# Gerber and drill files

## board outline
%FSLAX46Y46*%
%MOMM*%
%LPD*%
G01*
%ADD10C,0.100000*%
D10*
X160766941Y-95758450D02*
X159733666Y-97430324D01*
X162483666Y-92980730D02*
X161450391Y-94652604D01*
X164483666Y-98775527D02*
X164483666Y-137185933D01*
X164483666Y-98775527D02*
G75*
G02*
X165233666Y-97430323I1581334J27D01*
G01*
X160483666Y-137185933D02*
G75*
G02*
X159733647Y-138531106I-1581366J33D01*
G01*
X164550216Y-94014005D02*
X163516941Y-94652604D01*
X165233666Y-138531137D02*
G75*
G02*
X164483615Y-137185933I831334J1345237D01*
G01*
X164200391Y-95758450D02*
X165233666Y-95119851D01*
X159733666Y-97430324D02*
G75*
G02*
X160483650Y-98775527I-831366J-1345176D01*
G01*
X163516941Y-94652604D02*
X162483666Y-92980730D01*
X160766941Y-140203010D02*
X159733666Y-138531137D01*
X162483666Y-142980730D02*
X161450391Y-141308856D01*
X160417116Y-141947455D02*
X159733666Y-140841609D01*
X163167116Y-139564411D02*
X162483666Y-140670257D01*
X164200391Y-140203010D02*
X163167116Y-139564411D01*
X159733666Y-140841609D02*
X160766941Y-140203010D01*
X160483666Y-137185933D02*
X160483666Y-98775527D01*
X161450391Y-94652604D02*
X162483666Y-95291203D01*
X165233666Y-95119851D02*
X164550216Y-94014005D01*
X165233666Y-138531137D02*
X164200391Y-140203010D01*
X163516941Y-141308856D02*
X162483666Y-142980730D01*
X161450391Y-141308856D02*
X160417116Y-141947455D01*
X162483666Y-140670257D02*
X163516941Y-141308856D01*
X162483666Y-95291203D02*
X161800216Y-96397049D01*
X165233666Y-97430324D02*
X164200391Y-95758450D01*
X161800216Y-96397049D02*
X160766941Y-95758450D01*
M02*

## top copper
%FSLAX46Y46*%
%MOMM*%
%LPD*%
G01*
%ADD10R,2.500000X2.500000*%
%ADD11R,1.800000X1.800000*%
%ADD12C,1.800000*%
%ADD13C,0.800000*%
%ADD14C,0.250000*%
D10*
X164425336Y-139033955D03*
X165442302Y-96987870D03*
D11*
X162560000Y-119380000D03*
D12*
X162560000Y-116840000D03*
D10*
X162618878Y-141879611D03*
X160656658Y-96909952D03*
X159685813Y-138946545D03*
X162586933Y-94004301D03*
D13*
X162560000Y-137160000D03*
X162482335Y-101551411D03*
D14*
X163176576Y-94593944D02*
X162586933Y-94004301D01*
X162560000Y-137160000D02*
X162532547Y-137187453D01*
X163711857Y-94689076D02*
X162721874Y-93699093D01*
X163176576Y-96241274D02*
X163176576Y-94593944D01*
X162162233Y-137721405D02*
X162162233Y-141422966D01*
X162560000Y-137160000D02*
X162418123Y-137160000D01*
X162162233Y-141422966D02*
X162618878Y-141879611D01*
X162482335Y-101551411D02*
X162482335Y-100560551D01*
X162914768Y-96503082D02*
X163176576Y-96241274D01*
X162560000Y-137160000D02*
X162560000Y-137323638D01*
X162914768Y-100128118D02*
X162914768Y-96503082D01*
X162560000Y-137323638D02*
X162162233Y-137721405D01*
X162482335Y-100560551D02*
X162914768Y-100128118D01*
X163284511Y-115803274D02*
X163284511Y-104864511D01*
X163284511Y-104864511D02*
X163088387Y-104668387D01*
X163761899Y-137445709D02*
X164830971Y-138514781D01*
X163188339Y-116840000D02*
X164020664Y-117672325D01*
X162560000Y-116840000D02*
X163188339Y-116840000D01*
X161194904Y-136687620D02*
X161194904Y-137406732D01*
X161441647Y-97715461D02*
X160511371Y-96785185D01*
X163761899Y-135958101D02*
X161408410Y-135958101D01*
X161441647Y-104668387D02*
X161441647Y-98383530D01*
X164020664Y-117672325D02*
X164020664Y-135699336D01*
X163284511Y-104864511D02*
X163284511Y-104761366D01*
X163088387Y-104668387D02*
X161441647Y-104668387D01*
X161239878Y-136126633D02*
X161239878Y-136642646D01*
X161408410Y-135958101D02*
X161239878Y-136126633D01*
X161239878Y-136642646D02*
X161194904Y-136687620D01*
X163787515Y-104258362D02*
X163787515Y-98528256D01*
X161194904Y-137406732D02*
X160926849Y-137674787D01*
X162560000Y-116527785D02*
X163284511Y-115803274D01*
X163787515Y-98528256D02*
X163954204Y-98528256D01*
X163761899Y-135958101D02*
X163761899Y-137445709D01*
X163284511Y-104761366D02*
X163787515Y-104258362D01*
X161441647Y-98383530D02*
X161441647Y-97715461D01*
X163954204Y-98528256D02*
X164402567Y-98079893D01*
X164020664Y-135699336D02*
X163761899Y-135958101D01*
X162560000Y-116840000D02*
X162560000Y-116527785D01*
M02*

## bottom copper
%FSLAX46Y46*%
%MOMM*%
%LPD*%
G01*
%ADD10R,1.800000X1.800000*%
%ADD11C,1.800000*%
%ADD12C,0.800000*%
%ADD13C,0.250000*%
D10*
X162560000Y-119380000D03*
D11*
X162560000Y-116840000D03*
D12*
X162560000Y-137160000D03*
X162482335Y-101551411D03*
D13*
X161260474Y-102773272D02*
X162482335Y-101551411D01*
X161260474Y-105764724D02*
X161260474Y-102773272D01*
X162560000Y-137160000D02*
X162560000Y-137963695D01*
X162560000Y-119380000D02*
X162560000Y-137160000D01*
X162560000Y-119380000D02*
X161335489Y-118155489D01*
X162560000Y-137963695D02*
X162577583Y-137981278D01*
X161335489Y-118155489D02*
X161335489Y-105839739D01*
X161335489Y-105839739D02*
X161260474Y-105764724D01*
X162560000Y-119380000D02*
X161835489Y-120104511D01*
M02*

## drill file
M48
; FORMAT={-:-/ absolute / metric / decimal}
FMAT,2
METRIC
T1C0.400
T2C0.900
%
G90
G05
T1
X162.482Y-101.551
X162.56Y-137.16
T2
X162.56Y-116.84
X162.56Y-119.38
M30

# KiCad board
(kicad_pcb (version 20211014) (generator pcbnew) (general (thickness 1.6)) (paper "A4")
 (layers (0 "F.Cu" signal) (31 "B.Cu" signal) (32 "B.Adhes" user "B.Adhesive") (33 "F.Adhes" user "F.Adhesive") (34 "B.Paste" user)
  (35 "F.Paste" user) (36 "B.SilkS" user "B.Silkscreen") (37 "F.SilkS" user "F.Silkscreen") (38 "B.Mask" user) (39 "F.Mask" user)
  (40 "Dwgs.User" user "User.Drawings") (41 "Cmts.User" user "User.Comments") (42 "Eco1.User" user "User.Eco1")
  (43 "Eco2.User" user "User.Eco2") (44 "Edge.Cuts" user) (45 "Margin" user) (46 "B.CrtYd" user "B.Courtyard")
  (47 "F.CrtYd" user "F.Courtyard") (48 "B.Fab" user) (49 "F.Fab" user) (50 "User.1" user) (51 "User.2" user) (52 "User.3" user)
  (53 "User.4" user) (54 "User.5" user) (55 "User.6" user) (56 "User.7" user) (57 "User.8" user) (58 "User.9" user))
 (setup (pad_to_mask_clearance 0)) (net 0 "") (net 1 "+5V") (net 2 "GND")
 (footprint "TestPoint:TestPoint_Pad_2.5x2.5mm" (layer "F.Cu") (at 164.425336 139.033955)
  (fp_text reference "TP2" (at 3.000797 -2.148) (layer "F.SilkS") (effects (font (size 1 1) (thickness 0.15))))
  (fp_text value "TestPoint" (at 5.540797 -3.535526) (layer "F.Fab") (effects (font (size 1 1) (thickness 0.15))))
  (pad "1" smd rect (at 0 0) (size 2.5 2.5) (layers "F.Cu" "F.Mask") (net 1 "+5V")))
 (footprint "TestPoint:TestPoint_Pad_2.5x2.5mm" (layer "F.Cu") (at 165.442302 96.98787)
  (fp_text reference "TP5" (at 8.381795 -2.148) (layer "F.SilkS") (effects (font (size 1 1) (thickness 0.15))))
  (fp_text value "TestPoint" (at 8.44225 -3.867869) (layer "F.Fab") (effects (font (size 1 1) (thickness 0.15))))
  (pad "1" smd rect (at 0 0) (size 2.5 2.5) (layers "F.Cu" "F.Mask") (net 1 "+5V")))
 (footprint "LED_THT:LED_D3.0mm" (layer "F.Cu") (at 162.56 119.38 90)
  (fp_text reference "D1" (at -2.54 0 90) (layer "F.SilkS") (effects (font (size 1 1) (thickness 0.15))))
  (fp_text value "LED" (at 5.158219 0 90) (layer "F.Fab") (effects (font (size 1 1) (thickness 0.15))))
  (pad "1" thru_hole rect (at 0 0 90) (size 1.8 1.8) (drill 0.9) (layers *.Cu *.Mask) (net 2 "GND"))
  (pad "2" thru_hole circle (at 2.54 0 90) (size 1.8 1.8) (drill 0.9) (layers *.Cu *.Mask) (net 1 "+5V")))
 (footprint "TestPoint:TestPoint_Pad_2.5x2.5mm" (layer "F.Cu") (at 162.618878 141.879611)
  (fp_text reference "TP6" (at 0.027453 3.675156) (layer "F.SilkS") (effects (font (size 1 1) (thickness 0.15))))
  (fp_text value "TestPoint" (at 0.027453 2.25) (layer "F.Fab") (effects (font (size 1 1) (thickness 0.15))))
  (pad "1" smd rect (at 0 0) (size 2.5 2.5) (layers "F.Cu" "F.Mask") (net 2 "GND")))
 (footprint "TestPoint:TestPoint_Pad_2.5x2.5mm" (layer "F.Cu") (at 160.656658 96.909952)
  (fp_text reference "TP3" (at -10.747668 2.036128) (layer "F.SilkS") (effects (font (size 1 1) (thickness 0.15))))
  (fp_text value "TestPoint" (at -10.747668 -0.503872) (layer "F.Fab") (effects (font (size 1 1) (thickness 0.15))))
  (pad "1" smd rect (at 0 0) (size 2.5 2.5) (layers "F.Cu" "F.Mask") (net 1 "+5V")))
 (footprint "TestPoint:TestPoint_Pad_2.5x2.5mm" (layer "F.Cu") (at 159.685813 138.946545)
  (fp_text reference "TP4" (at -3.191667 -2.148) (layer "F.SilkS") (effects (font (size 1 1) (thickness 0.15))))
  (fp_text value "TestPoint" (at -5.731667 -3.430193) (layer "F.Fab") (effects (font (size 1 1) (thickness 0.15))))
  (pad "1" smd rect (at 0 0) (size 2.5 2.5) (layers "F.Cu" "F.Mask") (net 1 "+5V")))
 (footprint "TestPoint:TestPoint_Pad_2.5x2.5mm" (layer "F.Cu") (at 162.586933 94.004301)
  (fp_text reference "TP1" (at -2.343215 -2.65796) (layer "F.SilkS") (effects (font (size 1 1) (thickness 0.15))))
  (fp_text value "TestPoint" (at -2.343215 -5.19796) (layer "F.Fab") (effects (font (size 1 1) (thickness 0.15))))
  (pad "1" smd rect (at 0 0) (size 2.5 2.5) (layers "F.Cu" "F.Mask") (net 2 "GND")))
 (gr_line (start 160.766941 95.75845) (end 159.733666 97.430324) (layer "Edge.Cuts") (width 0.1))
 (gr_line (start 162.483666 92.98073) (end 161.450391 94.652604) (layer "Edge.Cuts") (width 0.1))
 (gr_line (start 164.483666 98.775527) (end 164.483666 137.185933) (layer "Edge.Cuts") (width 0.1))
 (gr_arc (start 164.483666 98.775527) (mid 164.683834 98.00545) (end 165.233666 97.430324) (layer "Edge.Cuts") (width 0.1))
 (gr_arc (start 160.483666 137.185933) (mid 160.283498 137.95601) (end 159.733666 138.531137) (layer "Edge.Cuts") (width 0.1))
 (gr_line (start 164.550216 94.014005) (end 163.516941 94.652604) (layer "Edge.Cuts") (width 0.1))
 (gr_arc (start 165.233666 138.531137) (mid 164.683834 137.95601) (end 164.483666 137.185933) (layer "Edge.Cuts") (width 0.1))
 (gr_line (start 164.200391 95.75845) (end 165.233666 95.119851) (layer "Edge.Cuts") (width 0.1))
 (gr_arc (start 159.733666 97.430324) (mid 160.283498 98.00545) (end 160.483666 98.775527) (layer "Edge.Cuts") (width 0.1))
 (gr_line (start 163.516941 94.652604) (end 162.483666 92.98073) (layer "Edge.Cuts") (width 0.1))
 (gr_line (start 160.766941 140.20301) (end 159.733666 138.531137) (layer "Edge.Cuts") (width 0.1))
 (gr_line (start 162.483666 142.98073) (end 161.450391 141.308856) (layer "Edge.Cuts") (width 0.1))
 (gr_line (start 160.417116 141.947455) (end 159.733666 140.841609) (layer "Edge.Cuts") (width 0.1))
 (gr_line (start 163.167116 139.564411) (end 162.483666 140.670257) (layer "Edge.Cuts") (width 0.1))
 (gr_line (start 164.200391 140.20301) (end 163.167116 139.564411) (layer "Edge.Cuts") (width 0.1))
 (gr_line (start 159.733666 140.841609) (end 160.766941 140.20301) (layer "Edge.Cuts") (width 0.1))
 (gr_line (start 160.483666 137.185933) (end 160.483666 98.775527) (layer "Edge.Cuts") (width 0.1))
 (gr_line (start 161.450391 94.652604) (end 162.483666 95.291203) (layer "Edge.Cuts") (width 0.1))
 (gr_line (start 165.233666 95.119851) (end 164.550216 94.014005) (layer "Edge.Cuts") (width 0.1))
 (gr_line (start 165.233666 138.531137) (end 164.200391 140.20301) (layer "Edge.Cuts") (width 0.1))
 (gr_line (start 163.516941 141.308856) (end 162.483666 142.98073) (layer "Edge.Cuts") (width 0.1))
 (gr_line (start 161.450391 141.308856) (end 160.417116 141.947455) (layer "Edge.Cuts") (width 0.1))
 (gr_line (start 162.483666 140.670257) (end 163.516941 141.308856) (layer "Edge.Cuts") (width 0.1))
 (gr_line (start 162.483666 95.291203) (end 161.800216 96.397049) (layer "Edge.Cuts") (width 0.1))
 (gr_line (start 165.233666 97.430324) (end 164.200391 95.75845) (layer "Edge.Cuts") (width 0.1))
 (gr_line (start 161.800216 96.397049) (end 160.766941 95.75845) (layer "Edge.Cuts") (width 0.1))
 (segment (start 163.176576 94.593944) (end 162.586933 94.004301) (width 0.25) (layer "F.Cu") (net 2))
 (segment (start 162.56 137.16) (end 162.532547 137.187453) (width 0.25) (layer "F.Cu") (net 2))
 (segment (start 163.711857 94.689076) (end 162.721874 93.699093) (width 0.25) (layer "F.Cu") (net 2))
 (segment (start 163.176576 96.241274) (end 163.176576 94.593944) (width 0.25) (layer "F.Cu") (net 2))
 (segment (start 162.162233 137.721405) (end 162.162233 141.422966) (width 0.25) (layer "F.Cu") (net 2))
 (segment (start 162.56 137.16) (end 162.418123 137.16) (width 0.25) (layer "F.Cu") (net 2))
 (segment (start 162.162233 141.422966) (end 162.618878 141.879611) (width 0.25) (layer "F.Cu") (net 2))
 (segment (start 162.482335 101.551411) (end 162.482335 100.560551) (width 0.25) (layer "F.Cu") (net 2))
 (segment (start 162.914768 96.503082) (end 163.176576 96.241274) (width 0.25) (layer "F.Cu") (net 2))
 (segment (start 162.56 137.16) (end 162.56 137.323638) (width 0.25) (layer "F.Cu") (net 2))
 (segment (start 162.914768 100.128118) (end 162.914768 96.503082) (width 0.25) (layer "F.Cu") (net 2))
 (segment (start 162.56 137.323638) (end 162.162233 137.721405) (width 0.25) (layer "F.Cu") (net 2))
 (segment (start 162.482335 100.560551) (end 162.914768 100.128118) (width 0.25) (layer "F.Cu") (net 2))
 (via (at 162.56 137.16) (size 0.8) (drill 0.4) (layers "F.Cu" "B.Cu") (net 2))
 (via (at 162.482335 101.551411) (size 0.8) (drill 0.4) (layers "F.Cu" "B.Cu") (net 2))
 (segment (start 161.260474 102.773272) (end 162.482335 101.551411) (width 0.25) (layer "B.Cu") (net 2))
 (segment (start 161.260474 105.764724) (end 161.260474 102.773272) (width 0.25) (layer "B.Cu") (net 2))
 (segment (start 162.56 137.16) (end 162.56 137.963695) (width 0.25) (layer "B.Cu") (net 2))
 (segment (start 162.56 119.38) (end 162.56 137.16) (width 0.25) (layer "B.Cu") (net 2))
 (segment (start 162.56 119.38) (end 161.335489 118.155489) (width 0.25) (layer "B.Cu") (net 2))
 (segment (start 162.56 137.963695) (end 162.577583 137.981278) (width 0.25) (layer "B.Cu") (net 2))
 (segment (start 161.335489 118.155489) (end 161.335489 105.839739) (width 0.25) (layer "B.Cu") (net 2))
 (segment (start 161.335489 105.839739) (end 161.260474 105.764724) (width 0.25) (layer "B.Cu") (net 2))
 (segment (start 162.56 119.38) (end 161.835489 120.104511) (width 0.25) (layer "B.Cu") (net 2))
 (segment (start 163.284511 115.803274) (end 163.284511 104.864511) (width 0.25) (layer "F.Cu") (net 1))
 (segment (start 163.284511 104.864511) (end 163.088387 104.668387) (width 0.25) (layer "F.Cu") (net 1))
 (segment (start 163.761899 137.445709) (end 164.830971 138.514781) (width 0.25) (layer "F.Cu") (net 1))
 (segment (start 163.188339 116.84) (end 164.020664 117.672325) (width 0.25) (layer "F.Cu") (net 1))
 (segment (start 162.56 116.84) (end 163.188339 116.84) (width 0.25) (layer "F.Cu") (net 1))
 (segment (start 161.194904 136.68762) (end 161.194904 137.406732) (width 0.25) (layer "F.Cu") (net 1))
 (segment (start 161.441647 97.715461) (end 160.511371 96.785185) (width 0.25) (layer "F.Cu") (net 1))
 (segment (start 163.761899 135.958101) (end 161.40841 135.958101) (width 0.25) (layer "F.Cu") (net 1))
 (segment (start 161.441647 104.668387) (end 161.441647 98.38353) (width 0.25) (layer "F.Cu") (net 1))
 (segment (start 164.020664 117.672325) (end 164.020664 135.699336) (width 0.25) (layer "F.Cu") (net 1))
 (segment (start 163.284511 104.864511) (end 163.284511 104.761366) (width 0.25) (layer "F.Cu") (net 1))
 (segment (start 163.088387 104.668387) (end 161.441647 104.668387) (width 0.25) (layer "F.Cu") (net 1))
 (segment (start 161.239878 136.126633) (end 161.239878 136.642646) (width 0.25) (layer "F.Cu") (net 1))
 (segment (start 161.40841 135.958101) (end 161.239878 136.126633) (width 0.25) (layer "F.Cu") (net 1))
 (segment (start 161.239878 136.642646) (end 161.194904 136.68762) (width 0.25) (layer "F.Cu") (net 1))
 (segment (start 163.787515 104.258362) (end 163.787515 98.528256) (width 0.25) (layer "F.Cu") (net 1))
 (segment (start 161.194904 137.406732) (end 160.926849 137.674787) (width 0.25) (layer "F.Cu") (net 1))
 (segment (start 162.56 116.527785) (end 163.284511 115.803274) (width 0.25) (layer "F.Cu") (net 1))
 (segment (start 163.787515 98.528256) (end 163.954204 98.528256) (width 0.25) (layer "F.Cu") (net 1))
 (segment (start 163.761899 135.958101) (end 163.761899 137.445709) (width 0.25) (layer "F.Cu") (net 1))
 (segment (start 163.284511 104.761366) (end 163.787515 104.258362) (width 0.25) (layer "F.Cu") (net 1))
 (segment (start 161.441647 98.38353) (end 161.441647 97.715461) (width 0.25) (layer "F.Cu") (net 1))
 (segment (start 163.954204 98.528256) (end 164.402567 98.079893) (width 0.25) (layer "F.Cu") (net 1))
 (segment (start 164.020664 135.699336) (end 163.761899 135.958101) (width 0.25) (layer "F.Cu") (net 1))
 (segment (start 162.56 116.84) (end 162.56 116.527785) (width 0.25) (layer "F.Cu") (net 1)))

